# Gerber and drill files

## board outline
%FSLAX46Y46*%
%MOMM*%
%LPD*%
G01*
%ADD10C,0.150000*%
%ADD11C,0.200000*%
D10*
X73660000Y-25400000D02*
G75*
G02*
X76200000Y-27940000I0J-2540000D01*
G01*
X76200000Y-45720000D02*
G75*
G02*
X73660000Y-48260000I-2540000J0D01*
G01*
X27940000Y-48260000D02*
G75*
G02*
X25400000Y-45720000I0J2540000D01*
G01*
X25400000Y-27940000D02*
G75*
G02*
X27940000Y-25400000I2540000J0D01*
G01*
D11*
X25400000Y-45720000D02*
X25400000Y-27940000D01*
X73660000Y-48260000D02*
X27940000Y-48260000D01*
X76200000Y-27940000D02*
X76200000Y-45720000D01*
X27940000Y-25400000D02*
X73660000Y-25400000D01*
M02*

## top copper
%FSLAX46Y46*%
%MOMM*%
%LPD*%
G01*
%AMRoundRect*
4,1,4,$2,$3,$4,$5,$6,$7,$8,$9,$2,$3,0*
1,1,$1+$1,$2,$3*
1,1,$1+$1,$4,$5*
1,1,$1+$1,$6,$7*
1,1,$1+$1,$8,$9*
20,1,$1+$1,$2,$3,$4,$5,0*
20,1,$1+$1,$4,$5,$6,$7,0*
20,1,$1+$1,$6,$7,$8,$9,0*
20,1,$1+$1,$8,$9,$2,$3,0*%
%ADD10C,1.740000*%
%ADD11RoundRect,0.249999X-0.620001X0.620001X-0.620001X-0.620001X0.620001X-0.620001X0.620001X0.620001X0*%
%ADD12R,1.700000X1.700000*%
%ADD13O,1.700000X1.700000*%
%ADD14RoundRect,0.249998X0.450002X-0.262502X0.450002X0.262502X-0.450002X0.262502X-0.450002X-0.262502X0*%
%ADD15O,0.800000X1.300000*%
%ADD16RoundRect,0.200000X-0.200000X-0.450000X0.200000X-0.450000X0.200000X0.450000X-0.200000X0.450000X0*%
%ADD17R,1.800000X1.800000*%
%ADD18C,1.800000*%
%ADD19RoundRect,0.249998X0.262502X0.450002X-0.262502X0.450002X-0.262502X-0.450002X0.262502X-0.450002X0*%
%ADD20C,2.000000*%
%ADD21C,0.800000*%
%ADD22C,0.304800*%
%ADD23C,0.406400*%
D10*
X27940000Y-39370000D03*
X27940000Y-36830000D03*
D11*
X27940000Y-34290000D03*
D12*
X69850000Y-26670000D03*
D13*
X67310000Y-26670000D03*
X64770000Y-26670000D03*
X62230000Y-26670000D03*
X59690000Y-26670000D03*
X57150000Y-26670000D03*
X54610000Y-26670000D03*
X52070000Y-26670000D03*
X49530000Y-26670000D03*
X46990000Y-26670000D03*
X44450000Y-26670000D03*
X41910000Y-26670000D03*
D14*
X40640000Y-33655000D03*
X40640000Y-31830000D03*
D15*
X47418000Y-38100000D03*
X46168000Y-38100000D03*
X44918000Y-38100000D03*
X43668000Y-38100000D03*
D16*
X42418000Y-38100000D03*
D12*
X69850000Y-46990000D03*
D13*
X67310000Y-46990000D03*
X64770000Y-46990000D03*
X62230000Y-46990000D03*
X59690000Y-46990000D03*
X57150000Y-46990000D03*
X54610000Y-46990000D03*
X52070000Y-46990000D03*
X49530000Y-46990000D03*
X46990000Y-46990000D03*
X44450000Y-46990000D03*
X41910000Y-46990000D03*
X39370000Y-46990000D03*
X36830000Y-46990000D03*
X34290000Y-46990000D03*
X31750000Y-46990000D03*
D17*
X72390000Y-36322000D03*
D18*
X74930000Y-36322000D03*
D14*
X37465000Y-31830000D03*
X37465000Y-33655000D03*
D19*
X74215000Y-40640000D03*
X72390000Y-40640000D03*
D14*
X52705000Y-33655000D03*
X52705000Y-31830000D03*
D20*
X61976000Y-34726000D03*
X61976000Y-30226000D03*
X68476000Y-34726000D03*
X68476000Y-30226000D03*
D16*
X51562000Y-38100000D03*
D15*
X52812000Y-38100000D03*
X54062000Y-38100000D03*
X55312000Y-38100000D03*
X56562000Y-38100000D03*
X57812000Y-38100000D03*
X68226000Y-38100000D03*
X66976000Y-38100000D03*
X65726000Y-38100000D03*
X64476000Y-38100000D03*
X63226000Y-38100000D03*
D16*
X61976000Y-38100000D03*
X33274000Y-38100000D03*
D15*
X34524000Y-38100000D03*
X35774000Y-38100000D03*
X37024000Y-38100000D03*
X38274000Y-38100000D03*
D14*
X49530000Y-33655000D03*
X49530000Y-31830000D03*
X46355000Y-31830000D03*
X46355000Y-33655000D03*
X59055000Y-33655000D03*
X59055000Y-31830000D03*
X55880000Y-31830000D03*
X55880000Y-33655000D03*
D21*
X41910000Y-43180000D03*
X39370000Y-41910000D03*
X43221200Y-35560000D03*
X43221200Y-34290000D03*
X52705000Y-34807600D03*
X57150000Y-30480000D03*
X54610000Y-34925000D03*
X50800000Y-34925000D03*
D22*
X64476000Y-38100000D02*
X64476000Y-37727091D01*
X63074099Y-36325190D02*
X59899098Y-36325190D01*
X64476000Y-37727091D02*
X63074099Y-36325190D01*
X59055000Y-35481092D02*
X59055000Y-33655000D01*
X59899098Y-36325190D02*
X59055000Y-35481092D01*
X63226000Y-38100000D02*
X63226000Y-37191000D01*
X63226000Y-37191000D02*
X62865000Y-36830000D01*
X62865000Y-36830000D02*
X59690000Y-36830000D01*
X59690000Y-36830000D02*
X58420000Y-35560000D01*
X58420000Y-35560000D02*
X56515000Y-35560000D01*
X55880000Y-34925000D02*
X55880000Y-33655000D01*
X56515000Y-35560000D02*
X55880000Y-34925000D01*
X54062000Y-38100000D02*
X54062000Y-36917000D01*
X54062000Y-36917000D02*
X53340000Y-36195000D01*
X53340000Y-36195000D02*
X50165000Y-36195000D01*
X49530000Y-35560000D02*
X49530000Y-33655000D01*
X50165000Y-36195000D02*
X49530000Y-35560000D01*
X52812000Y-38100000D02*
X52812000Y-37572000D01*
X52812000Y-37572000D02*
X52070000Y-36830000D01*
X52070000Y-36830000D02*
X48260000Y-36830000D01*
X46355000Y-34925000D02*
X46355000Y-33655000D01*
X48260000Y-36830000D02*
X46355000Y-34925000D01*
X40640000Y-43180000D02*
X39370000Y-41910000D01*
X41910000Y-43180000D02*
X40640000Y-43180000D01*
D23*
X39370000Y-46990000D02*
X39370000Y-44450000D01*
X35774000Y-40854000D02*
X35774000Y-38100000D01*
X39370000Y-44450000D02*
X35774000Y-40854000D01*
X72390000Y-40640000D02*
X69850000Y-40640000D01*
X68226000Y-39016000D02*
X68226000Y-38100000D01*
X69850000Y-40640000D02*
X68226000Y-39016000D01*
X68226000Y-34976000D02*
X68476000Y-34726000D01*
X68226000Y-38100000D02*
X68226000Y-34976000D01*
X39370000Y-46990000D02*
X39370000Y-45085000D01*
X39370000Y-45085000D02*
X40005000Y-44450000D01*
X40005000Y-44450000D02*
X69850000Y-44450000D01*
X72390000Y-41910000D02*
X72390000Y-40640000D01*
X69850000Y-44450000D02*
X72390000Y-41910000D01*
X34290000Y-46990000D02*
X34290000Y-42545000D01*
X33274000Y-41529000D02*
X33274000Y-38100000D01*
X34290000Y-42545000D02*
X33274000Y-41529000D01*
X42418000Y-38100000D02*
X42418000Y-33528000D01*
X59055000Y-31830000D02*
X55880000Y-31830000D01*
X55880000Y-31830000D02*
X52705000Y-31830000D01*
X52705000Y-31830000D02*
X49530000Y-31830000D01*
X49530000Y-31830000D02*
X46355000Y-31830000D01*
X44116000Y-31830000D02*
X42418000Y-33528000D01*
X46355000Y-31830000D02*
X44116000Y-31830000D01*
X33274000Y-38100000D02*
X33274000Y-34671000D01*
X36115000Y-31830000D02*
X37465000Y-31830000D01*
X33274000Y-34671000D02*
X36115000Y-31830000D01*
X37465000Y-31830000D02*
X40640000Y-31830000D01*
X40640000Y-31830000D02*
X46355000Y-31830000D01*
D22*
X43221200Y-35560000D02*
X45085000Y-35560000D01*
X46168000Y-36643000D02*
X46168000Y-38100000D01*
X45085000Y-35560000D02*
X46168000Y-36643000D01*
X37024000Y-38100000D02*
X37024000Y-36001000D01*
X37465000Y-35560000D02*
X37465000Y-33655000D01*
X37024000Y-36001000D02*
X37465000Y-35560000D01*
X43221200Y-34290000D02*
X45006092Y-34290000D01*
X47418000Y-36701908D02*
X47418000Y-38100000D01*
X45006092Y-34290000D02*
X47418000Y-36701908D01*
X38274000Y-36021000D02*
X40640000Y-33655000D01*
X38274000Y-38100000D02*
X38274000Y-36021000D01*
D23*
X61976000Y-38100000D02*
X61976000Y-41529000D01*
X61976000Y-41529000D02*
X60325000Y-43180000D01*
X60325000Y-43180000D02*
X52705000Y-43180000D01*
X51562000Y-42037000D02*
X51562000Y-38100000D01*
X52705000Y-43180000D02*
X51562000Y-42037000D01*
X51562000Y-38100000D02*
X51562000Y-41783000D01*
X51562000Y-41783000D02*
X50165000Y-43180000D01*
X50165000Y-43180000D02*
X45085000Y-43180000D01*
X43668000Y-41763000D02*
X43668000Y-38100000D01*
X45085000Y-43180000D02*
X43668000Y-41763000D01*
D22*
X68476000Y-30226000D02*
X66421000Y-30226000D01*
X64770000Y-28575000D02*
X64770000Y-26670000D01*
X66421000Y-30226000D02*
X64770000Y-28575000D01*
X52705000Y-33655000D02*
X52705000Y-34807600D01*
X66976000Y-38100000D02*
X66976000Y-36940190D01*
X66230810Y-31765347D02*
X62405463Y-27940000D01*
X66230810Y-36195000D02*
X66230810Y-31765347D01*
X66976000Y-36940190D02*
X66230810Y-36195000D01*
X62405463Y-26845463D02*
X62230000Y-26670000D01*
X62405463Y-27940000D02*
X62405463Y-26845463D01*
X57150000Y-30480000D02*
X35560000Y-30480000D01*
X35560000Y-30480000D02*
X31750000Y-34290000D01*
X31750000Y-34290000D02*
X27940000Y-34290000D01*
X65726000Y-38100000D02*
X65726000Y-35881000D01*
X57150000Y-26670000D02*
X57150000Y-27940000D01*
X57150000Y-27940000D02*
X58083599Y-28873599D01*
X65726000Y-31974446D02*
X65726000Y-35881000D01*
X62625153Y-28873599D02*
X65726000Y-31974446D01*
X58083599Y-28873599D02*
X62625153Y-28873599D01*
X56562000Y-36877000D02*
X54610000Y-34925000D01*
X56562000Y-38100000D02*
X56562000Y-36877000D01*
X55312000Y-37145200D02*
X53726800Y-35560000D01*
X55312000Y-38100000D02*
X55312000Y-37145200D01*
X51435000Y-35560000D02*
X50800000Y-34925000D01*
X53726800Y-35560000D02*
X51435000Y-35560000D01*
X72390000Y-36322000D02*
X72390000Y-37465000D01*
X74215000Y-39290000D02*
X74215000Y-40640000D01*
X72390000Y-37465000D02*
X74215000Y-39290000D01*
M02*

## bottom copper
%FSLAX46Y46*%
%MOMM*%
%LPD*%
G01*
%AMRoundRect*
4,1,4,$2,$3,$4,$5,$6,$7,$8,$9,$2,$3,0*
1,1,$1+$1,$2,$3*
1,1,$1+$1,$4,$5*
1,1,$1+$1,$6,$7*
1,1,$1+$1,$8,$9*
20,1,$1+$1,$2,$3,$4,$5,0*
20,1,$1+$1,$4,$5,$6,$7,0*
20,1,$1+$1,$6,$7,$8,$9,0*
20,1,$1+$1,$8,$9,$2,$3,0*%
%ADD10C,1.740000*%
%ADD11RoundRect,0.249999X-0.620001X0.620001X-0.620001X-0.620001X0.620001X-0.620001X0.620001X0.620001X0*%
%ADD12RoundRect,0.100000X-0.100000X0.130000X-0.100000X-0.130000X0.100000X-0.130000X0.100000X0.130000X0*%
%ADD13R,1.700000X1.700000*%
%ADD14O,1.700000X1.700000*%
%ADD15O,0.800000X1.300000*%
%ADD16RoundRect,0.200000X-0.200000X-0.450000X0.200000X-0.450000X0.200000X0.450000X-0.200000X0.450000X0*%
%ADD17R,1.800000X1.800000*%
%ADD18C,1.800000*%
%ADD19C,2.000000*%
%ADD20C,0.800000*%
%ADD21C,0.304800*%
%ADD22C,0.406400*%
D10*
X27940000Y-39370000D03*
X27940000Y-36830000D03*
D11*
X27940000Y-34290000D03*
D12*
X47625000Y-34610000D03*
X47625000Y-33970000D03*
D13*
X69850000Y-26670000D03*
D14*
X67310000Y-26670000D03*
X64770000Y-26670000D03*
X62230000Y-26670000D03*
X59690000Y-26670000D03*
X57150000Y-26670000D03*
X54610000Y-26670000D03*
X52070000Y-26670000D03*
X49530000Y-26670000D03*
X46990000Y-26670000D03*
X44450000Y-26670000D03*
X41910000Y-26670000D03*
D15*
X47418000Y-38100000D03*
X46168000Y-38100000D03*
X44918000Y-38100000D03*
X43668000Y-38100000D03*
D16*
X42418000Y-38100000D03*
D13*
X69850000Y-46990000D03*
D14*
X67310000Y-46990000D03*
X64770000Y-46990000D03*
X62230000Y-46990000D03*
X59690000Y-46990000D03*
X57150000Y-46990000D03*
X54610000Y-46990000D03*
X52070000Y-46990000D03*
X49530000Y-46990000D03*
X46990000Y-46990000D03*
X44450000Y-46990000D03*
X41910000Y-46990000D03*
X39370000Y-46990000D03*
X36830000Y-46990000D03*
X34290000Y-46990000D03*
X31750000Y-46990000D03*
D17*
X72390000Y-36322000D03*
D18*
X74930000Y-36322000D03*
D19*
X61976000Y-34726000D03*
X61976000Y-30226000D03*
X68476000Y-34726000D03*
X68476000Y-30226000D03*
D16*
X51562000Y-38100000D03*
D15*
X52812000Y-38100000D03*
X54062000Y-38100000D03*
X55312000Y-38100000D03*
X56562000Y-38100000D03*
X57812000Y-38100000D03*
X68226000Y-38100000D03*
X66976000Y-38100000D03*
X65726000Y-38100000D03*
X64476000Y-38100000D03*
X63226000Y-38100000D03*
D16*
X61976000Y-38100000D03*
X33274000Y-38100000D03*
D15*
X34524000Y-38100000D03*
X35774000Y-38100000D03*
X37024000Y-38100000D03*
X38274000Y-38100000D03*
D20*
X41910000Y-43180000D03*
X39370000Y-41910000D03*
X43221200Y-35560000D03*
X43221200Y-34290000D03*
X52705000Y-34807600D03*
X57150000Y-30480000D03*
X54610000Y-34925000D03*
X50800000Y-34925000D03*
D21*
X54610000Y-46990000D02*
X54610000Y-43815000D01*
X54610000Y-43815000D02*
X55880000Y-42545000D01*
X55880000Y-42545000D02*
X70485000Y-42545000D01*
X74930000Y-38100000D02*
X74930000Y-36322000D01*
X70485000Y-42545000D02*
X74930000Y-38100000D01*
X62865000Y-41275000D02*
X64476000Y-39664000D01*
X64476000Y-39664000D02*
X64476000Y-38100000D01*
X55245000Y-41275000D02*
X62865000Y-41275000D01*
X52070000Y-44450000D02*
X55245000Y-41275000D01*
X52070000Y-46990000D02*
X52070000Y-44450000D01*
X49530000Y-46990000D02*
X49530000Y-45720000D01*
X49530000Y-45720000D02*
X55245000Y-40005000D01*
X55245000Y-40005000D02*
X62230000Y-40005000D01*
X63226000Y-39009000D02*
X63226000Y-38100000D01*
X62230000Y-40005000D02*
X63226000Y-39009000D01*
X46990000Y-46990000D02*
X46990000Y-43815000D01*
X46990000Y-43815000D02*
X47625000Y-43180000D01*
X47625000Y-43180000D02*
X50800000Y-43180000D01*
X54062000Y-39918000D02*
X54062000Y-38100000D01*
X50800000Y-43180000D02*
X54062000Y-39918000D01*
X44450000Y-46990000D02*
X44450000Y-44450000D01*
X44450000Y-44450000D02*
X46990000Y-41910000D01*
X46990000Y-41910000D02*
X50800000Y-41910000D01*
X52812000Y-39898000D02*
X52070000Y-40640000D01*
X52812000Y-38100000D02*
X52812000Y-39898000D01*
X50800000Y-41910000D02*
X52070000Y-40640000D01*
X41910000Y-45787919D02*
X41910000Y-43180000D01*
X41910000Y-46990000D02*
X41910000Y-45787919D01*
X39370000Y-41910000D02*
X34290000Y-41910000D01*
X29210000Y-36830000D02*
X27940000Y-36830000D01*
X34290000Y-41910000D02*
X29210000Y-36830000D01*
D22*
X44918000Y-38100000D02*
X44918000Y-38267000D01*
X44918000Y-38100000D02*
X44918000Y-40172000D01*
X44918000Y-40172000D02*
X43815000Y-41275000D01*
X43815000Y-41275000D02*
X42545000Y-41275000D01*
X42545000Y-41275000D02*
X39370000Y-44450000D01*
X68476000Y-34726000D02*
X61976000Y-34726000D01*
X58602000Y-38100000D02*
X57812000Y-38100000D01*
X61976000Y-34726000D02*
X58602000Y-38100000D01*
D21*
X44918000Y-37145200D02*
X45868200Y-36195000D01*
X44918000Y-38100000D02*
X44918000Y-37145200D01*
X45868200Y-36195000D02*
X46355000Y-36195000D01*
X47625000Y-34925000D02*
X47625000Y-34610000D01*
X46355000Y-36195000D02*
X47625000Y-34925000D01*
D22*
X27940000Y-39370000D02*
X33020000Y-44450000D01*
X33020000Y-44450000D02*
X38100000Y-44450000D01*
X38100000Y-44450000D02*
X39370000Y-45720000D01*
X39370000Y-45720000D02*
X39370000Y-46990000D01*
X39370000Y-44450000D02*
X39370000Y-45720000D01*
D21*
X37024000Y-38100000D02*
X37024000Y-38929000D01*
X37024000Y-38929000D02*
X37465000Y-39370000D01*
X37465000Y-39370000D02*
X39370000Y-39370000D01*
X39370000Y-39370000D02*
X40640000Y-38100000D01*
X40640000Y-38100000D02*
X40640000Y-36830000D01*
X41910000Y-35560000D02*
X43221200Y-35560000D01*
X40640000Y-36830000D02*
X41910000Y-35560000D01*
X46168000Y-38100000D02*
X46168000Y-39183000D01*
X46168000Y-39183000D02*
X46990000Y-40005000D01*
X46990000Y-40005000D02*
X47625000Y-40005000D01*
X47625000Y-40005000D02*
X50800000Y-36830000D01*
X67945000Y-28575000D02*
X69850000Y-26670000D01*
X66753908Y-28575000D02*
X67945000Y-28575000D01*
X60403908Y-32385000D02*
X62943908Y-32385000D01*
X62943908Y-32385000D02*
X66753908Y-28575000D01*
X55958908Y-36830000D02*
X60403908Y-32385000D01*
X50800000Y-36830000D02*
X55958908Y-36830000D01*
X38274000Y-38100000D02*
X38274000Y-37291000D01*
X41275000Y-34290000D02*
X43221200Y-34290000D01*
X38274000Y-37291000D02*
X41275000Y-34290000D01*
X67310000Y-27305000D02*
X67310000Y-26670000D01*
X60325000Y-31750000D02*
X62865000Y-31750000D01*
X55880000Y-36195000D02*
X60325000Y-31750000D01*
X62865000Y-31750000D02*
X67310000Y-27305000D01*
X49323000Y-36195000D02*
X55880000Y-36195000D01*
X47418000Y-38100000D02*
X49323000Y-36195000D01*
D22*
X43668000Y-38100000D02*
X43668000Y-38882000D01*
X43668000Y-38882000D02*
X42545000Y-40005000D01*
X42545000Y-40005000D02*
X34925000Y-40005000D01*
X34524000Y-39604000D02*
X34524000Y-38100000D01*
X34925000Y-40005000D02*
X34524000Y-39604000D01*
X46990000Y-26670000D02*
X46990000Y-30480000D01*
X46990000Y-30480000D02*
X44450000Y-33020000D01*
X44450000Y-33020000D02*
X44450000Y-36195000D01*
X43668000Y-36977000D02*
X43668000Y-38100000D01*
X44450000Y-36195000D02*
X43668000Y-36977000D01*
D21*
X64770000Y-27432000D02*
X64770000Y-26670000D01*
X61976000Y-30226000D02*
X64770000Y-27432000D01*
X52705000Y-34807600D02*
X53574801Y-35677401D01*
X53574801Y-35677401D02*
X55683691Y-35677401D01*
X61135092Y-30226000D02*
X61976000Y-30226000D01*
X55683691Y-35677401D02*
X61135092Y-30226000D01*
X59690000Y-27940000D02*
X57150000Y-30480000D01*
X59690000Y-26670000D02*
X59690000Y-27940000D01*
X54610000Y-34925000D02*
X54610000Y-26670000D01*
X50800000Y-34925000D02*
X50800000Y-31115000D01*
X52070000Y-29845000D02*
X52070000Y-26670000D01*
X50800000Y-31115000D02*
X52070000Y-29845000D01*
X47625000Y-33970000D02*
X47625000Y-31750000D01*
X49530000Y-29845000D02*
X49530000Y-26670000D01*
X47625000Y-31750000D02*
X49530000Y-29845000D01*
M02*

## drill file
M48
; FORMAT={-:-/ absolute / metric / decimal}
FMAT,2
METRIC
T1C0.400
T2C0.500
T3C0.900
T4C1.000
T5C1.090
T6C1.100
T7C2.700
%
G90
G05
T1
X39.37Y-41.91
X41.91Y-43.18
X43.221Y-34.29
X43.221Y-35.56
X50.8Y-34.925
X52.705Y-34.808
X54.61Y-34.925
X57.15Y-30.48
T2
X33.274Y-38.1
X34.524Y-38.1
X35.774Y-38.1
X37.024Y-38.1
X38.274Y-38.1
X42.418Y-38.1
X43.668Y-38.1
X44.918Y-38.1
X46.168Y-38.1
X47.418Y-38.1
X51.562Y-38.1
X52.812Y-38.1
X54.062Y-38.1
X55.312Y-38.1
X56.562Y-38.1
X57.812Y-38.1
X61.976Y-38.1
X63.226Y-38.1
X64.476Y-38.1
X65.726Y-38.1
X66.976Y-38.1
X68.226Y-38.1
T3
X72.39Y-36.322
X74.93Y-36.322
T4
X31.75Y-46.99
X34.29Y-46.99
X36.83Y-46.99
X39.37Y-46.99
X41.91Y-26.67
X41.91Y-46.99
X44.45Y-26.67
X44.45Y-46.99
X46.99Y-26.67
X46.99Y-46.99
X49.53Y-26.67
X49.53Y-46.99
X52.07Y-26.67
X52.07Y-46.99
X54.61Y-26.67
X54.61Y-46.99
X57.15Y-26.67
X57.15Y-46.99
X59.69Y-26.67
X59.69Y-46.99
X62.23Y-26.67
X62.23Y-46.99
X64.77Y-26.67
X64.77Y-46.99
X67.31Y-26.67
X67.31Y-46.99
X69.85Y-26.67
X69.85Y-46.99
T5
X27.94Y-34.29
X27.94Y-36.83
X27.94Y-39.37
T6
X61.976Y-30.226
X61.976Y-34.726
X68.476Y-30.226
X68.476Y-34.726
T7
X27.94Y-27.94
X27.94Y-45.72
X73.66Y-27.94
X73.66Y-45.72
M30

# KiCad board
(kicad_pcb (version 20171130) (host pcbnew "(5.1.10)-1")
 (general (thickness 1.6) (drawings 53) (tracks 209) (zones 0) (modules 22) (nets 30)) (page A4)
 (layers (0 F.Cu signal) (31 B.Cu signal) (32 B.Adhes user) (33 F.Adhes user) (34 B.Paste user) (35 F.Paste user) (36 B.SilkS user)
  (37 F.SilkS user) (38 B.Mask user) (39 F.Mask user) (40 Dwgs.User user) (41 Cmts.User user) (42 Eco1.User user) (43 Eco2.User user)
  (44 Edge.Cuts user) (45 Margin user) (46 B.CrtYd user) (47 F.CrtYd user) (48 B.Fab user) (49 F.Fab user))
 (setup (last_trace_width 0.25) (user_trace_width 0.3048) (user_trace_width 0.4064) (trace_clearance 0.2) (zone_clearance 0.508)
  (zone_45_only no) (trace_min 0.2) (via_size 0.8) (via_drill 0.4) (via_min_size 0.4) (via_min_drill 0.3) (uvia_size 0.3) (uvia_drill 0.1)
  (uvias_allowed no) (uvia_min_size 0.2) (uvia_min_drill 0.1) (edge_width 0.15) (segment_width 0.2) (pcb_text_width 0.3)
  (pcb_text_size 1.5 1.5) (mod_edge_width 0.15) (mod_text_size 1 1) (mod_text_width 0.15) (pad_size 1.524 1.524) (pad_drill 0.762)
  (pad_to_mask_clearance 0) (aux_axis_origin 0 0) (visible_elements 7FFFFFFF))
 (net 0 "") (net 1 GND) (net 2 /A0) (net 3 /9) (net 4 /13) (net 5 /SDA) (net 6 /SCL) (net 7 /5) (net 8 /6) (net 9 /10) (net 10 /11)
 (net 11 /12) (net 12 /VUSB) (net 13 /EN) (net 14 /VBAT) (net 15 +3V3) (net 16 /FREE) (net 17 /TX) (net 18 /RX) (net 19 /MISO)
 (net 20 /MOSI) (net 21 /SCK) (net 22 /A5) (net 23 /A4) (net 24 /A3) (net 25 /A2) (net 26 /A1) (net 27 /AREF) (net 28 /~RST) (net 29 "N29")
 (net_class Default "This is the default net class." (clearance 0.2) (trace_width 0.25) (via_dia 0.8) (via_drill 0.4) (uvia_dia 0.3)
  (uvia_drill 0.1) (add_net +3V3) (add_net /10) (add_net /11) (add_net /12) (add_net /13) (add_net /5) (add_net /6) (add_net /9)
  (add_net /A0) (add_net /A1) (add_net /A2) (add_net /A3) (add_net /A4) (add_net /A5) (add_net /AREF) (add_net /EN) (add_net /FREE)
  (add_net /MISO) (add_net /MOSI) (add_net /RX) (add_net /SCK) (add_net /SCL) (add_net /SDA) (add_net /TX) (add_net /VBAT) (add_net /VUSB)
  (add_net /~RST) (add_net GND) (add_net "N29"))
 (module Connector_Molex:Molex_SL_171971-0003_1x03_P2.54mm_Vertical (layer F.Cu) (at 27.94 34.29 270)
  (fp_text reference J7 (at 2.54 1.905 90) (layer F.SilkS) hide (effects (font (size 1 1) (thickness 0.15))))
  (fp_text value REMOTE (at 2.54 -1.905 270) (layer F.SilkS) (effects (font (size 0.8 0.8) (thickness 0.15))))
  (pad 3 thru_hole circle (at 5.08 0 270) (size 1.74 1.74) (drill 1.09) (layers *.Cu *.Mask) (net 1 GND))
  (pad 2 thru_hole circle (at 2.54 0 270) (size 1.74 1.74) (drill 1.09) (layers *.Cu *.Mask) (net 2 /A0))
  (pad 1 thru_hole roundrect (at 0 0 270) (size 1.74 1.74) (drill 1.09) (layers *.Cu *.Mask) (roundrect_rratio 0.1436775862068966)
   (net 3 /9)))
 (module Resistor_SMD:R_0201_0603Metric (layer B.Cu) (at 47.625 34.29 270)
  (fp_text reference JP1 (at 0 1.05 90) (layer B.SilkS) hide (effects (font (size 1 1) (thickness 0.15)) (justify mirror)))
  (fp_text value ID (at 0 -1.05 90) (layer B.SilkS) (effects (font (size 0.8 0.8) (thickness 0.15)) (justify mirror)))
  (pad 2 smd roundrect (at 0.32 0 270) (size 0.46 0.4) (layers B.Cu B.Mask) (roundrect_rratio 0.25) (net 1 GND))
  (pad 1 smd roundrect (at -0.32 0 270) (size 0.46 0.4) (layers B.Cu B.Mask) (roundrect_rratio 0.25) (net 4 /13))
  (pad "" smd roundrect (at 0.345 0 270) (size 0.318 0.36) (layers B.Paste) (roundrect_rratio 0.25))
  (pad "" smd roundrect (at -0.345 0 270) (size 0.318 0.36) (layers B.Paste) (roundrect_rratio 0.25)))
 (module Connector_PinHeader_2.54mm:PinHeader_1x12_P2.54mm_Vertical (layer B.Cu) (at 69.85 26.67 90)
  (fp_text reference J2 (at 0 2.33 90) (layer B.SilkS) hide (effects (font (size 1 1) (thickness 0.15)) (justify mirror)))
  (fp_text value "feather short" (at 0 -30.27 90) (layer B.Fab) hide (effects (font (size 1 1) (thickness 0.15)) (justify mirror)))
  (pad 1 thru_hole rect (at 0 0 90) (size 1.7 1.7) (drill 1) (layers *.Cu *.Mask) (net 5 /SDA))
  (pad 2 thru_hole oval (at 0 -2.54 90) (size 1.7 1.7) (drill 1) (layers *.Cu *.Mask) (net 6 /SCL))
  (pad 3 thru_hole oval (at 0 -5.08 90) (size 1.7 1.7) (drill 1) (layers *.Cu *.Mask) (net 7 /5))
  (pad 4 thru_hole oval (at 0 -7.62 90) (size 1.7 1.7) (drill 1) (layers *.Cu *.Mask) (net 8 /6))
  (pad 5 thru_hole oval (at 0 -10.16 90) (size 1.7 1.7) (drill 1) (layers *.Cu *.Mask) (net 3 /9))
  (pad 6 thru_hole oval (at 0 -12.7 90) (size 1.7 1.7) (drill 1) (layers *.Cu *.Mask) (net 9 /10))
  (pad 7 thru_hole oval (at 0 -15.24 90) (size 1.7 1.7) (drill 1) (layers *.Cu *.Mask) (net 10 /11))
  (pad 8 thru_hole oval (at 0 -17.78 90) (size 1.7 1.7) (drill 1) (layers *.Cu *.Mask) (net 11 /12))
  (pad 9 thru_hole oval (at 0 -20.32 90) (size 1.7 1.7) (drill 1) (layers *.Cu *.Mask) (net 4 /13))
  (pad 10 thru_hole oval (at 0 -22.86 90) (size 1.7 1.7) (drill 1) (layers *.Cu *.Mask) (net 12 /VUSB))
  (pad 11 thru_hole oval (at 0 -25.4 90) (size 1.7 1.7) (drill 1) (layers *.Cu *.Mask) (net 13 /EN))
  (pad 12 thru_hole oval (at 0 -27.94 90) (size 1.7 1.7) (drill 1) (layers *.Cu *.Mask) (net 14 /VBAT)))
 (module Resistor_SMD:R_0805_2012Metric (layer F.Cu) (at 40.64 32.7425 90)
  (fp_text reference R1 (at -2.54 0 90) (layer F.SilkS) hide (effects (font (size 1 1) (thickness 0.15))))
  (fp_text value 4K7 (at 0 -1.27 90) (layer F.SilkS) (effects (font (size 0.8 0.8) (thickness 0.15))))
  (pad 1 smd roundrect (at -0.9125 0 90) (size 1.025 1.4) (layers F.Cu F.Paste F.Mask) (roundrect_rratio 0.2439004878048781) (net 6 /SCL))
  (pad 2 smd roundrect (at 0.9125 0 90) (size 1.025 1.4) (layers F.Cu F.Paste F.Mask) (roundrect_rratio 0.2439004878048781) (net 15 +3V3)))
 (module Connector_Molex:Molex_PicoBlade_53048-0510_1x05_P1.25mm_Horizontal (layer F.Cu) (at 42.418 38.1)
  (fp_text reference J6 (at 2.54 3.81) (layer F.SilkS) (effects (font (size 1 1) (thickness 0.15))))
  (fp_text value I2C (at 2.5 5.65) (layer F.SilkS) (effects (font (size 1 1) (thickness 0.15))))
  (pad 5 thru_hole oval (at 5 0) (size 0.8 1.3) (drill 0.5) (layers *.Cu *.Mask) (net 6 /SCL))
  (pad 4 thru_hole oval (at 3.75 0) (size 0.8 1.3) (drill 0.5) (layers *.Cu *.Mask) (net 5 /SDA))
  (pad 3 thru_hole oval (at 2.5 0) (size 0.8 1.3) (drill 0.5) (layers *.Cu *.Mask) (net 1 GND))
  (pad 2 thru_hole oval (at 1.25 0) (size 0.8 1.3) (drill 0.5) (layers *.Cu *.Mask) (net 12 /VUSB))
  (pad 1 thru_hole roundrect (at 0 0) (size 0.8 1.3) (drill 0.5) (layers *.Cu *.Mask) (roundrect_rratio 0.25) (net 15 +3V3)))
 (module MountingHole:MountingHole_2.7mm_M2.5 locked (layer F.Cu) (at 73.66 27.94)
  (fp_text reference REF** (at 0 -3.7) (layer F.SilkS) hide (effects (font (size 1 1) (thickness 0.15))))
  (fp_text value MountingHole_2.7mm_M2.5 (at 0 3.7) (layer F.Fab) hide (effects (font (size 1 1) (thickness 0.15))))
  (pad 1 np_thru_hole circle (at 0 0) (size 2.7 2.7) (drill 2.7) (layers *.Cu *.Mask)))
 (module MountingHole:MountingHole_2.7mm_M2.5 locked (layer F.Cu) (at 73.66 45.72)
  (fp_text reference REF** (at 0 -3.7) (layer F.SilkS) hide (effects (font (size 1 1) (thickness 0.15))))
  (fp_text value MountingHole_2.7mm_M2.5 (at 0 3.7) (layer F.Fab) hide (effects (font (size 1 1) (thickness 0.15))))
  (pad 1 np_thru_hole circle (at 0 0) (size 2.7 2.7) (drill 2.7) (layers *.Cu *.Mask)))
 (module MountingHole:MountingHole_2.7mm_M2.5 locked (layer F.Cu) (at 27.94 45.72)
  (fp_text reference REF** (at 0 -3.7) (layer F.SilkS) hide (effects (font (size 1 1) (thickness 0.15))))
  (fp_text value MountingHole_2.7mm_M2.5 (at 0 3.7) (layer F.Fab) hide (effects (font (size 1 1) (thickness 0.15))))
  (pad 1 np_thru_hole circle (at 0 0) (size 2.7 2.7) (drill 2.7) (layers *.Cu *.Mask)))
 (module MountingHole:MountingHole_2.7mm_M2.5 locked (layer F.Cu) (at 27.94 27.94)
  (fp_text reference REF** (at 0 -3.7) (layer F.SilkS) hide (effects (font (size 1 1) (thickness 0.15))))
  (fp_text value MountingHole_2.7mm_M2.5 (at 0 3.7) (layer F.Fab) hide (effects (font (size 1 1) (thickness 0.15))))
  (pad 1 np_thru_hole circle (at 0 0) (size 2.7 2.7) (drill 2.7) (layers *.Cu *.Mask)))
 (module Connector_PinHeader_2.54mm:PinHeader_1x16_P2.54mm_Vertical (layer B.Cu) (at 69.85 46.99 90)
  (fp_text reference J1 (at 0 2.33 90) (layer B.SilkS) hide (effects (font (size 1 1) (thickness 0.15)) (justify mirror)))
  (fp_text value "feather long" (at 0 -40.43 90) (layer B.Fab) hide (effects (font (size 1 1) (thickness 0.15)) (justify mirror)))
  (pad 1 thru_hole rect (at 0 0 90) (size 1.7 1.7) (drill 1) (layers *.Cu *.Mask) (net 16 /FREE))
  (pad 2 thru_hole oval (at 0 -2.54 90) (size 1.7 1.7) (drill 1) (layers *.Cu *.Mask) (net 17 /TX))
  (pad 3 thru_hole oval (at 0 -5.08 90) (size 1.7 1.7) (drill 1) (layers *.Cu *.Mask) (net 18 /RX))
  (pad 4 thru_hole oval (at 0 -7.62 90) (size 1.7 1.7) (drill 1) (layers *.Cu *.Mask) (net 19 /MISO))
  (pad 5 thru_hole oval (at 0 -10.16 90) (size 1.7 1.7) (drill 1) (layers *.Cu *.Mask) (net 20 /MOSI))
  (pad 6 thru_hole oval (at 0 -12.7 90) (size 1.7 1.7) (drill 1) (layers *.Cu *.Mask) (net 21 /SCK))
  (pad 7 thru_hole oval (at 0 -15.24 90) (size 1.7 1.7) (drill 1) (layers *.Cu *.Mask) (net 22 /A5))
  (pad 8 thru_hole oval (at 0 -17.78 90) (size 1.7 1.7) (drill 1) (layers *.Cu *.Mask) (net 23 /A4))
  (pad 9 thru_hole oval (at 0 -20.32 90) (size 1.7 1.7) (drill 1) (layers *.Cu *.Mask) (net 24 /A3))
  (pad 10 thru_hole oval (at 0 -22.86 90) (size 1.7 1.7) (drill 1) (layers *.Cu *.Mask) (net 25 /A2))
  (pad 11 thru_hole oval (at 0 -25.4 90) (size 1.7 1.7) (drill 1) (layers *.Cu *.Mask) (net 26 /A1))
  (pad 12 thru_hole oval (at 0 -27.94 90) (size 1.7 1.7) (drill 1) (layers *.Cu *.Mask) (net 2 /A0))
  (pad 13 thru_hole oval (at 0 -30.48 90) (size 1.7 1.7) (drill 1) (layers *.Cu *.Mask) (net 1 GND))
  (pad 14 thru_hole oval (at 0 -33.02 90) (size 1.7 1.7) (drill 1) (layers *.Cu *.Mask) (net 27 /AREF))
  (pad 15 thru_hole oval (at 0 -35.56 90) (size 1.7 1.7) (drill 1) (layers *.Cu *.Mask) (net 15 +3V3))
  (pad 16 thru_hole oval (at 0 -38.1 90) (size 1.7 1.7) (drill 1) (layers *.Cu *.Mask) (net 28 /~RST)))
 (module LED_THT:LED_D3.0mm (layer F.Cu) (at 72.39 36.322)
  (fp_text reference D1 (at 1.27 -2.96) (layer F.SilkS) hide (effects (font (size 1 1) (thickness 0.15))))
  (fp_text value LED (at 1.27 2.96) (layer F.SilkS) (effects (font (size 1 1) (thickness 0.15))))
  (pad 1 thru_hole rect (at 0 0) (size 1.8 1.8) (drill 0.9) (layers *.Cu *.Mask) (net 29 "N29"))
  (pad 2 thru_hole circle (at 2.54 0) (size 1.8 1.8) (drill 0.9) (layers *.Cu *.Mask) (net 22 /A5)))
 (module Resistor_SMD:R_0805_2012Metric (layer F.Cu) (at 37.465 32.7425 90)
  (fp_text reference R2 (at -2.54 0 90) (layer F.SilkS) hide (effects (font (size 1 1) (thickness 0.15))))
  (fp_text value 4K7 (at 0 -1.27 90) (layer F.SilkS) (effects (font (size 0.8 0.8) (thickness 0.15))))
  (pad 2 smd roundrect (at 0.9125 0 90) (size 1.025 1.4) (layers F.Cu F.Paste F.Mask) (roundrect_rratio 0.2439004878048781) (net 15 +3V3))
  (pad 1 smd roundrect (at -0.9125 0 90) (size 1.025 1.4) (layers F.Cu F.Paste F.Mask) (roundrect_rratio 0.2439004878048781) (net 5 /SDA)))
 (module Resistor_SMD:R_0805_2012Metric (layer F.Cu) (at 73.3025 40.64 180)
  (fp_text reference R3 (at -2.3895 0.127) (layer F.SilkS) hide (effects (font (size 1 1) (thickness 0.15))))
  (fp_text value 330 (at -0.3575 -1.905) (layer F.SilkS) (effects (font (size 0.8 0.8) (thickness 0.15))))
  (pad 1 smd roundrect (at -0.9125 0 180) (size 1.025 1.4) (layers F.Cu F.Paste F.Mask) (roundrect_rratio 0.2439004878048781) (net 29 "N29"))
  (pad 2 smd roundrect (at 0.9125 0 180) (size 1.025 1.4) (layers F.Cu F.Paste F.Mask) (roundrect_rratio 0.2439004878048781) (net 1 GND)))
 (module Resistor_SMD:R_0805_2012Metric (layer F.Cu) (at 52.705 32.7425 90)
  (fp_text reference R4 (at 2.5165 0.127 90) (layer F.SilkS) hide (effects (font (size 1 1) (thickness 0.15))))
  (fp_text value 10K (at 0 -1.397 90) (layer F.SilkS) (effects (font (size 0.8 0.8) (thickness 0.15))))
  (pad 1 smd roundrect (at -0.9125 0 90) (size 1.025 1.4) (layers F.Cu F.Paste F.Mask) (roundrect_rratio 0.2439004878048781) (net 7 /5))
  (pad 2 smd roundrect (at 0.9125 0 90) (size 1.025 1.4) (layers F.Cu F.Paste F.Mask) (roundrect_rratio 0.2439004878048781) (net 15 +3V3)))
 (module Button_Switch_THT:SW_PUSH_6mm (layer F.Cu) (at 61.976 30.226)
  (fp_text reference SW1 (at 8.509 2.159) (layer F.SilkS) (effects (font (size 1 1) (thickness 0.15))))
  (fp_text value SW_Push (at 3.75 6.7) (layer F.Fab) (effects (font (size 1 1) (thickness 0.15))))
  (pad 2 thru_hole circle (at 0 4.5 90) (size 2 2) (drill 1.1) (layers *.Cu *.Mask) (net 1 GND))
  (pad 1 thru_hole circle (at 0 0 90) (size 2 2) (drill 1.1) (layers *.Cu *.Mask) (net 7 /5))
  (pad 2 thru_hole circle (at 6.5 4.5 90) (size 2 2) (drill 1.1) (layers *.Cu *.Mask) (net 1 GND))
  (pad 1 thru_hole circle (at 6.5 0 90) (size 2 2) (drill 1.1) (layers *.Cu *.Mask) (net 7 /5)))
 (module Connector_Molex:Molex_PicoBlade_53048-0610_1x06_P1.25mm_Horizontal (layer F.Cu) (at 51.562 38.1)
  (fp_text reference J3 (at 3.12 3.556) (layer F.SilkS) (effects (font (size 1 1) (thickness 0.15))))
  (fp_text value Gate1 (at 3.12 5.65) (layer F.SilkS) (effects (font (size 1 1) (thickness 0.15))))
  (pad 1 thru_hole roundrect (at 0 0) (size 0.8 1.3) (drill 0.5) (layers *.Cu *.Mask) (roundrect_rratio 0.25) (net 12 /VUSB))
  (pad 2 thru_hole oval (at 1.25 0) (size 0.8 1.3) (drill 0.5) (layers *.Cu *.Mask) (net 26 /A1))
  (pad 3 thru_hole oval (at 2.5 0) (size 0.8 1.3) (drill 0.5) (layers *.Cu *.Mask) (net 25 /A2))
  (pad 4 thru_hole oval (at 3.75 0) (size 0.8 1.3) (drill 0.5) (layers *.Cu *.Mask) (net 11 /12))
  (pad 5 thru_hole oval (at 5 0) (size 0.8 1.3) (drill 0.5) (layers *.Cu *.Mask) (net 10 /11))
  (pad 6 thru_hole oval (at 6.25 0) (size 0.8 1.3) (drill 0.5) (layers *.Cu *.Mask) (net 1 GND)))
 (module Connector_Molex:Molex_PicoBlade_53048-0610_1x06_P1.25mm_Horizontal (layer F.Cu) (at 61.976 38.1)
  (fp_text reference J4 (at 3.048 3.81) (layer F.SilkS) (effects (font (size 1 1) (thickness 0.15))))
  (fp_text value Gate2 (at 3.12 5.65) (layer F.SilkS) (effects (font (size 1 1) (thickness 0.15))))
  (pad 6 thru_hole oval (at 6.25 0) (size 0.8 1.3) (drill 0.5) (layers *.Cu *.Mask) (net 1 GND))
  (pad 5 thru_hole oval (at 5 0) (size 0.8 1.3) (drill 0.5) (layers *.Cu *.Mask) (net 8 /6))
  (pad 4 thru_hole oval (at 3.75 0) (size 0.8 1.3) (drill 0.5) (layers *.Cu *.Mask) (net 9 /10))
  (pad 3 thru_hole oval (at 2.5 0) (size 0.8 1.3) (drill 0.5) (layers *.Cu *.Mask) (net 23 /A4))
  (pad 2 thru_hole oval (at 1.25 0) (size 0.8 1.3) (drill 0.5) (layers *.Cu *.Mask) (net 24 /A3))
  (pad 1 thru_hole roundrect (at 0 0) (size 0.8 1.3) (drill 0.5) (layers *.Cu *.Mask) (roundrect_rratio 0.25) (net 12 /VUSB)))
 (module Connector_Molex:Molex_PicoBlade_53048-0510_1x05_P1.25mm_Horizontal (layer F.Cu) (at 33.274 38.1)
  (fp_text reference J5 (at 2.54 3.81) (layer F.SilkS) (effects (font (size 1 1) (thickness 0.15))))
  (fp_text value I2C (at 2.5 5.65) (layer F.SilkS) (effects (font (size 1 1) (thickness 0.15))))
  (pad 1 thru_hole roundrect (at 0 0) (size 0.8 1.3) (drill 0.5) (layers *.Cu *.Mask) (roundrect_rratio 0.25) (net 15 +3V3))
  (pad 2 thru_hole oval (at 1.25 0) (size 0.8 1.3) (drill 0.5) (layers *.Cu *.Mask) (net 12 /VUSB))
  (pad 3 thru_hole oval (at 2.5 0) (size 0.8 1.3) (drill 0.5) (layers *.Cu *.Mask) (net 1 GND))
  (pad 4 thru_hole oval (at 3.75 0) (size 0.8 1.3) (drill 0.5) (layers *.Cu *.Mask) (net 5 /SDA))
  (pad 5 thru_hole oval (at 5 0) (size 0.8 1.3) (drill 0.5) (layers *.Cu *.Mask) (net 6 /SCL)))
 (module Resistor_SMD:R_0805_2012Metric (layer F.Cu) (at 49.53 32.7425 90)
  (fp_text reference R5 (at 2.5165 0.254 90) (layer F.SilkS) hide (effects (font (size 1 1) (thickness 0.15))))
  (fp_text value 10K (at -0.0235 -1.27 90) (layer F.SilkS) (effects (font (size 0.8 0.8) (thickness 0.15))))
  (pad 1 smd roundrect (at -0.9125 0 90) (size 1.025 1.4) (layers F.Cu F.Paste F.Mask) (roundrect_rratio 0.2439004878048781) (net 25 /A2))
  (pad 2 smd roundrect (at 0.9125 0 90) (size 1.025 1.4) (layers F.Cu F.Paste F.Mask) (roundrect_rratio 0.2439004878048781) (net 15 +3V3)))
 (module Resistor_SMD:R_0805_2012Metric (layer F.Cu) (at 46.355 32.7425 90)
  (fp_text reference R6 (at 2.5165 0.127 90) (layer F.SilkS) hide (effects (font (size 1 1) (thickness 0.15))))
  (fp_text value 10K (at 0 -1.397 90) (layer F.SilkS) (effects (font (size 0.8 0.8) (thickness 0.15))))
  (pad 2 smd roundrect (at 0.9125 0 90) (size 1.025 1.4) (layers F.Cu F.Paste F.Mask) (roundrect_rratio 0.2439004878048781) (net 15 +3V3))
  (pad 1 smd roundrect (at -0.9125 0 90) (size 1.025 1.4) (layers F.Cu F.Paste F.Mask) (roundrect_rratio 0.2439004878048781) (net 26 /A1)))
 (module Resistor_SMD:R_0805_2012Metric (layer F.Cu) (at 59.055 32.7425 90)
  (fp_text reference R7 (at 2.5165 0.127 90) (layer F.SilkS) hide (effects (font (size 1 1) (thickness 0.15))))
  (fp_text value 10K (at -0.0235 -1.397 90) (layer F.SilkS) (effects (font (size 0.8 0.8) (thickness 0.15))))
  (pad 1 smd roundrect (at -0.9125 0 90) (size 1.025 1.4) (layers F.Cu F.Paste F.Mask) (roundrect_rratio 0.2439004878048781) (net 23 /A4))
  (pad 2 smd roundrect (at 0.9125 0 90) (size 1.025 1.4) (layers F.Cu F.Paste F.Mask) (roundrect_rratio 0.2439004878048781) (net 15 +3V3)))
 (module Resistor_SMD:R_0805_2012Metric (layer F.Cu) (at 55.88 32.7425 90)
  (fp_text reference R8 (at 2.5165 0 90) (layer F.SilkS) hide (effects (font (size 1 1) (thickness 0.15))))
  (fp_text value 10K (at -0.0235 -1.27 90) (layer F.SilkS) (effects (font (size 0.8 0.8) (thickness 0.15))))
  (pad 2 smd roundrect (at 0.9125 0 90) (size 1.025 1.4) (layers F.Cu F.Paste F.Mask) (roundrect_rratio 0.2439004878048781) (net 15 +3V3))
  (pad 1 smd roundrect (at -0.9125 0 90) (size 1.025 1.4) (layers F.Cu F.Paste F.Mask) (roundrect_rratio 0.2439004878048781) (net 24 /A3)))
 (gr_arc (start 73.66 27.94) (end 76.2 27.94) (angle -90) (layer Edge.Cuts) (width 0.15))
 (gr_arc (start 73.66 45.72) (end 73.66 48.26) (angle -90) (layer Edge.Cuts) (width 0.15))
 (gr_arc (start 27.94 45.72) (end 25.4 45.72) (angle -90) (layer Edge.Cuts) (width 0.15))
 (gr_arc (start 27.94 27.94) (end 27.94 25.4) (angle -90) (layer Edge.Cuts) (width 0.15))
 (gr_line (start 25.4 45.72) (end 25.4 27.94) (layer Edge.Cuts) (width 0.2))
 (gr_line (start 73.66 48.26) (end 27.94 48.26) (layer Edge.Cuts) (width 0.2))
 (gr_line (start 76.2 27.94) (end 76.2 45.72) (layer Edge.Cuts) (width 0.2))
 (gr_line (start 27.94 25.4) (end 73.66 25.4) (layer Edge.Cuts) (width 0.2))
 (segment (start 54.61 46.99) (end 54.61 43.815) (width 0.3048) (layer B.Cu) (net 22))
 (segment (start 54.61 43.815) (end 55.88 42.545) (width 0.3048) (layer B.Cu) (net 22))
 (segment (start 55.88 42.545) (end 70.485 42.545) (width 0.3048) (layer B.Cu) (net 22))
 (segment (start 74.93 38.1) (end 74.93 36.322) (width 0.3048) (layer B.Cu) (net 22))
 (segment (start 70.485 42.545) (end 74.93 38.1) (width 0.3048) (layer B.Cu) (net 22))
 (segment (start 62.865 41.275) (end 64.476 39.664) (width 0.3048) (layer B.Cu) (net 23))
 (segment (start 64.476 39.664) (end 64.476 38.1) (width 0.3048) (layer B.Cu) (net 23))
 (segment (start 55.245 41.275) (end 62.865 41.275) (width 0.3048) (layer B.Cu) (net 23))
 (segment (start 52.07 44.45) (end 55.245 41.275) (width 0.3048) (layer B.Cu) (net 23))
 (segment (start 52.07 46.99) (end 52.07 44.45) (width 0.3048) (layer B.Cu) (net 23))
 (segment (start 64.476 38.1) (end 64.476 37.727091) (width 0.3048) (layer F.Cu) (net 23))
 (segment (start 63.074099 36.32519) (end 59.899098 36.32519) (width 0.3048) (layer F.Cu) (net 23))
 (segment (start 64.476 37.727091) (end 63.074099 36.32519) (width 0.3048) (layer F.Cu) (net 23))
 (segment (start 59.055 35.481092) (end 59.055 33.655) (width 0.3048) (layer F.Cu) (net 23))
 (segment (start 59.899098 36.32519) (end 59.055 35.481092) (width 0.3048) (layer F.Cu) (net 23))
 (segment (start 49.53 46.99) (end 49.53 45.72) (width 0.3048) (layer B.Cu) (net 24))
 (segment (start 49.53 45.72) (end 55.245 40.005) (width 0.3048) (layer B.Cu) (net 24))
 (segment (start 55.245 40.005) (end 62.23 40.005) (width 0.3048) (layer B.Cu) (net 24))
 (segment (start 63.226 39.009) (end 63.226 38.1) (width 0.3048) (layer B.Cu) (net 24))
 (segment (start 62.23 40.005) (end 63.226 39.009) (width 0.3048) (layer B.Cu) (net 24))
 (segment (start 63.226 38.1) (end 63.226 37.191) (width 0.3048) (layer F.Cu) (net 24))
 (segment (start 63.226 37.191) (end 62.865 36.83) (width 0.3048) (layer F.Cu) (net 24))
 (segment (start 62.865 36.83) (end 59.69 36.83) (width 0.3048) (layer F.Cu) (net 24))
 (segment (start 59.69 36.83) (end 58.42 35.56) (width 0.3048) (layer F.Cu) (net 24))
 (segment (start 58.42 35.56) (end 56.515 35.56) (width 0.3048) (layer F.Cu) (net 24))
 (segment (start 55.88 34.925) (end 55.88 33.655) (width 0.3048) (layer F.Cu) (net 24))
 (segment (start 56.515 35.56) (end 55.88 34.925) (width 0.3048) (layer F.Cu) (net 24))
 (segment (start 46.99 46.99) (end 46.99 43.815) (width 0.3048) (layer B.Cu) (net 25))
 (segment (start 46.99 43.815) (end 47.625 43.18) (width 0.3048) (layer B.Cu) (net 25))
 (segment (start 47.625 43.18) (end 50.8 43.18) (width 0.3048) (layer B.Cu) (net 25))
 (segment (start 54.062 39.918) (end 54.062 38.1) (width 0.3048) (layer B.Cu) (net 25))
 (segment (start 50.8 43.18) (end 54.062 39.918) (width 0.3048) (layer B.Cu) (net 25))
 (segment (start 54.062 38.1) (end 54.062 36.917) (width 0.3048) (layer F.Cu) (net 25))
 (segment (start 54.062 36.917) (end 53.34 36.195) (width 0.3048) (layer F.Cu) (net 25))
 (segment (start 53.34 36.195) (end 50.165 36.195) (width 0.3048) (layer F.Cu) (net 25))
 (segment (start 49.53 35.56) (end 49.53 33.655) (width 0.3048) (layer F.Cu) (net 25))
 (segment (start 50.165 36.195) (end 49.53 35.56) (width 0.3048) (layer F.Cu) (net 25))
 (segment (start 44.45 46.99) (end 44.45 44.45) (width 0.3048) (layer B.Cu) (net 26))
 (segment (start 44.45 44.45) (end 46.99 41.91) (width 0.3048) (layer B.Cu) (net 26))
 (segment (start 46.99 41.91) (end 50.8 41.91) (width 0.3048) (layer B.Cu) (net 26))
 (segment (start 52.812 38.1) (end 52.812 37.572) (width 0.3048) (layer F.Cu) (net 26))
 (segment (start 52.812 37.572) (end 52.07 36.83) (width 0.3048) (layer F.Cu) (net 26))
 (segment (start 52.07 36.83) (end 48.26 36.83) (width 0.3048) (layer F.Cu) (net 26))
 (segment (start 46.355 34.925) (end 46.355 33.655) (width 0.3048) (layer F.Cu) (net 26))
 (segment (start 48.26 36.83) (end 46.355 34.925) (width 0.3048) (layer F.Cu) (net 26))
 (segment (start 52.812 39.898) (end 52.07 40.64) (width 0.3048) (layer B.Cu) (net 26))
 (segment (start 52.812 38.1) (end 52.812 39.898) (width 0.3048) (layer B.Cu) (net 26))
 (segment (start 50.8 41.91) (end 52.07 40.64) (width 0.3048) (layer B.Cu) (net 26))
 (via (at 41.91 43.18) (size 0.8) (drill 0.4) (layers F.Cu B.Cu) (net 2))
 (segment (start 41.91 45.787919) (end 41.91 43.18) (width 0.3048) (layer B.Cu) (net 2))
 (segment (start 41.91 46.99) (end 41.91 45.787919) (width 0.3048) (layer B.Cu) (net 2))
 (via (at 39.37 41.91) (size 0.8) (drill 0.4) (layers F.Cu B.Cu) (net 2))
 (segment (start 40.64 43.18) (end 39.37 41.91) (width 0.3048) (layer F.Cu) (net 2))
 (segment (start 41.91 43.18) (end 40.64 43.18) (width 0.3048) (layer F.Cu) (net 2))
 (segment (start 39.37 41.91) (end 34.29 41.91) (width 0.3048) (layer B.Cu) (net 2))
 (segment (start 29.21 36.83) (end 27.94 36.83) (width 0.3048) (layer B.Cu) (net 2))
 (segment (start 34.29 41.91) (end 29.21 36.83) (width 0.3048) (layer B.Cu) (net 2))
 (segment (start 39.37 46.99) (end 39.37 44.45) (width 0.4064) (layer F.Cu) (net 1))
 (segment (start 35.774 40.854) (end 35.774 38.1) (width 0.4064) (layer F.Cu) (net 1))
 (segment (start 39.37 44.45) (end 35.774 40.854) (width 0.4064) (layer F.Cu) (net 1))
 (segment (start 72.39 40.64) (end 69.85 40.64) (width 0.4064) (layer F.Cu) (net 1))
 (segment (start 68.226 39.016) (end 68.226 38.1) (width 0.4064) (layer F.Cu) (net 1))
 (segment (start 69.85 40.64) (end 68.226 39.016) (width 0.4064) (layer F.Cu) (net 1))
 (segment (start 68.226 34.976) (end 68.476 34.726) (width 0.4064) (layer F.Cu) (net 1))
 (segment (start 68.226 38.1) (end 68.226 34.976) (width 0.4064) (layer F.Cu) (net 1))
 (segment (start 44.918 38.1) (end 44.918 38.267) (width 0.4064) (layer B.Cu) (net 1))
 (segment (start 44.918 38.1) (end 44.918 40.172) (width 0.4064) (layer B.Cu) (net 1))
 (segment (start 44.918 40.172) (end 43.815 41.275) (width 0.4064) (layer B.Cu) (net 1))
 (segment (start 43.815 41.275) (end 42.545 41.275) (width 0.4064) (layer B.Cu) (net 1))
 (segment (start 42.545 41.275) (end 39.37 44.45) (width 0.4064) (layer B.Cu) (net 1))
 (segment (start 39.37 46.99) (end 39.37 45.085) (width 0.4064) (layer F.Cu) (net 1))
 (segment (start 39.37 45.085) (end 40.005 44.45) (width 0.4064) (layer F.Cu) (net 1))
 (segment (start 40.005 44.45) (end 69.85 44.45) (width 0.4064) (layer F.Cu) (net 1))
 (segment (start 72.39 41.91) (end 72.39 40.64) (width 0.4064) (layer F.Cu) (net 1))
 (segment (start 69.85 44.45) (end 72.39 41.91) (width 0.4064) (layer F.Cu) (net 1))
 (segment (start 68.476 34.726) (end 61.976 34.726) (width 0.4064) (layer B.Cu) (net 1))
 (segment (start 58.602 38.1) (end 57.812 38.1) (width 0.4064) (layer B.Cu) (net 1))
 (segment (start 61.976 34.726) (end 58.602 38.1) (width 0.4064) (layer B.Cu) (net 1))
 (segment (start 44.918 37.1452) (end 45.8682 36.195) (width 0.3048) (layer B.Cu) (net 1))
 (segment (start 44.918 38.1) (end 44.918 37.1452) (width 0.3048) (layer B.Cu) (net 1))
 (segment (start 45.8682 36.195) (end 46.355 36.195) (width 0.3048) (layer B.Cu) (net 1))
 (segment (start 47.625 34.925) (end 47.625 34.61) (width 0.3048) (layer B.Cu) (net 1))
 (segment (start 46.355 36.195) (end 47.625 34.925) (width 0.3048) (layer B.Cu) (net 1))
 (segment (start 27.94 39.37) (end 33.02 44.45) (width 0.4064) (layer B.Cu) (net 1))
 (segment (start 33.02 44.45) (end 38.1 44.45) (width 0.4064) (layer B.Cu) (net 1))
 (segment (start 38.1 44.45) (end 39.37 45.72) (width 0.4064) (layer B.Cu) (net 1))
 (segment (start 39.37 45.72) (end 39.37 46.99) (width 0.4064) (layer B.Cu) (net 1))
 (segment (start 39.37 44.45) (end 39.37 45.72) (width 0.4064) (layer B.Cu) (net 1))
 (segment (start 34.29 46.99) (end 34.29 42.545) (width 0.4064) (layer F.Cu) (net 15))
 (segment (start 33.274 41.529) (end 33.274 38.1) (width 0.4064) (layer F.Cu) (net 15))
 (segment (start 34.29 42.545) (end 33.274 41.529) (width 0.4064) (layer F.Cu) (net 15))
 (segment (start 42.418 38.1) (end 42.418 33.528) (width 0.4064) (layer F.Cu) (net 15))
 (segment (start 59.055 31.83) (end 55.88 31.83) (width 0.4064) (layer F.Cu) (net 15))
 (segment (start 55.88 31.83) (end 52.705 31.83) (width 0.4064) (layer F.Cu) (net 15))
 (segment (start 52.705 31.83) (end 49.53 31.83) (width 0.4064) (layer F.Cu) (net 15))
 (segment (start 49.53 31.83) (end 46.355 31.83) (width 0.4064) (layer F.Cu) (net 15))
 (segment (start 44.116 31.83) (end 42.418 33.528) (width 0.4064) (layer F.Cu) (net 15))
 (segment (start 46.355 31.83) (end 44.116 31.83) (width 0.4064) (layer F.Cu) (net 15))
 (segment (start 33.274 38.1) (end 33.274 34.671) (width 0.4064) (layer F.Cu) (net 15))
 (segment (start 36.115 31.83) (end 37.465 31.83) (width 0.4064) (layer F.Cu) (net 15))
 (segment (start 33.274 34.671) (end 36.115 31.83) (width 0.4064) (layer F.Cu) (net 15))
 (segment (start 37.465 31.83) (end 40.64 31.83) (width 0.4064) (layer F.Cu) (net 15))
 (segment (start 40.64 31.83) (end 46.355 31.83) (width 0.4064) (layer F.Cu) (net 15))
 (via (at 43.2212 35.56) (size 0.8) (drill 0.4) (layers F.Cu B.Cu) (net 5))
 (segment (start 43.2212 35.56) (end 45.085 35.56) (width 0.3048) (layer F.Cu) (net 5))
 (segment (start 46.168 36.643) (end 46.168 38.1) (width 0.3048) (layer F.Cu) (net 5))
 (segment (start 45.085 35.56) (end 46.168 36.643) (width 0.3048) (layer F.Cu) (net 5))
 (segment (start 37.024 38.1) (end 37.024 38.929) (width 0.3048) (layer B.Cu) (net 5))
 (segment (start 37.024 38.929) (end 37.465 39.37) (width 0.3048) (layer B.Cu) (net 5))
 (segment (start 37.465 39.37) (end 39.37 39.37) (width 0.3048) (layer B.Cu) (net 5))
 (segment (start 39.37 39.37) (end 40.64 38.1) (width 0.3048) (layer B.Cu) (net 5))
 (segment (start 40.64 38.1) (end 40.64 36.83) (width 0.3048) (layer B.Cu) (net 5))
 (segment (start 41.91 35.56) (end 43.2212 35.56) (width 0.3048) (layer B.Cu) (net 5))
 (segment (start 40.64 36.83) (end 41.91 35.56) (width 0.3048) (layer B.Cu) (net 5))
 (segment (start 46.168 38.1) (end 46.168 39.183) (width 0.3048) (layer B.Cu) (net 5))
 (segment (start 46.168 39.183) (end 46.99 40.005) (width 0.3048) (layer B.Cu) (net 5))
 (segment (start 46.99 40.005) (end 47.625 40.005) (width 0.3048) (layer B.Cu) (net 5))
 (segment (start 47.625 40.005) (end 50.8 36.83) (width 0.3048) (layer B.Cu) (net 5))
 (segment (start 67.945 28.575) (end 69.85 26.67) (width 0.3048) (layer B.Cu) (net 5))
 (segment (start 66.753908 28.575) (end 67.945 28.575) (width 0.3048) (layer B.Cu) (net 5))
 (segment (start 60.403908 32.385) (end 62.943908 32.385) (width 0.3048) (layer B.Cu) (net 5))
 (segment (start 62.943908 32.385) (end 66.753908 28.575) (width 0.3048) (layer B.Cu) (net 5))
 (segment (start 55.958908 36.83) (end 60.403908 32.385) (width 0.3048) (layer B.Cu) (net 5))
 (segment (start 50.8 36.83) (end 55.958908 36.83) (width 0.3048) (layer B.Cu) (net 5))
 (segment (start 37.024 38.1) (end 37.024 36.001) (width 0.3048) (layer F.Cu) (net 5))
 (segment (start 37.465 35.56) (end 37.465 33.655) (width 0.3048) (layer F.Cu) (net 5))
 (segment (start 37.024 36.001) (end 37.465 35.56) (width 0.3048) (layer F.Cu) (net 5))
 (segment (start 38.274 38.1) (end 38.274 37.291) (width 0.3048) (layer B.Cu) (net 6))
 (segment (start 41.275 34.29) (end 43.2212 34.29) (width 0.3048) (layer B.Cu) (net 6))
 (via (at 43.2212 34.29) (size 0.8) (drill 0.4) (layers F.Cu B.Cu) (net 6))
 (segment (start 38.274 37.291) (end 41.275 34.29) (width 0.3048) (layer B.Cu) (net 6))
 (segment (start 43.2212 34.29) (end 45.006092 34.29) (width 0.3048) (layer F.Cu) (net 6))
 (segment (start 47.418 36.701908) (end 47.418 38.1) (width 0.3048) (layer F.Cu) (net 6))
 (segment (start 45.006092 34.29) (end 47.418 36.701908) (width 0.3048) (layer F.Cu) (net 6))
 (segment (start 67.31 27.305) (end 67.31 26.67) (width 0.3048) (layer B.Cu) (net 6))
 (segment (start 60.325 31.75) (end 62.865 31.75) (width 0.3048) (layer B.Cu) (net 6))
 (segment (start 55.88 36.195) (end 60.325 31.75) (width 0.3048) (layer B.Cu) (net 6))
 (segment (start 62.865 31.75) (end 67.31 27.305) (width 0.3048) (layer B.Cu) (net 6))
 (segment (start 49.323 36.195) (end 55.88 36.195) (width 0.3048) (layer B.Cu) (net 6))
 (segment (start 47.418 38.1) (end 49.323 36.195) (width 0.3048) (layer B.Cu) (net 6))
 (segment (start 38.274 36.021) (end 40.64 33.655) (width 0.3048) (layer F.Cu) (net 6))
 (segment (start 38.274 38.1) (end 38.274 36.021) (width 0.3048) (layer F.Cu) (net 6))
 (segment (start 61.976 38.1) (end 61.976 41.529) (width 0.4064) (layer F.Cu) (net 12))
 (segment (start 61.976 41.529) (end 60.325 43.18) (width 0.4064) (layer F.Cu) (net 12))
 (segment (start 60.325 43.18) (end 52.705 43.18) (width 0.4064) (layer F.Cu) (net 12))
 (segment (start 51.562 42.037) (end 51.562 38.1) (width 0.4064) (layer F.Cu) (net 12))
 (segment (start 52.705 43.18) (end 51.562 42.037) (width 0.4064) (layer F.Cu) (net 12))
 (segment (start 51.562 38.1) (end 51.562 41.783) (width 0.4064) (layer F.Cu) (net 12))
 (segment (start 51.562 41.783) (end 50.165 43.18) (width 0.4064) (layer F.Cu) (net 12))
 (segment (start 50.165 43.18) (end 45.085 43.18) (width 0.4064) (layer F.Cu) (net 12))
 (segment (start 43.668 41.763) (end 43.668 38.1) (width 0.4064) (layer F.Cu) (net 12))
 (segment (start 45.085 43.18) (end 43.668 41.763) (width 0.4064) (layer F.Cu) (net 12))
 (segment (start 43.668 38.1) (end 43.668 38.882) (width 0.4064) (layer B.Cu) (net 12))
 (segment (start 43.668 38.882) (end 42.545 40.005) (width 0.4064) (layer B.Cu) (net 12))
 (segment (start 42.545 40.005) (end 34.925 40.005) (width 0.4064) (layer B.Cu) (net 12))
 (segment (start 34.524 39.604) (end 34.524 38.1) (width 0.4064) (layer B.Cu) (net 12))
 (segment (start 34.925 40.005) (end 34.524 39.604) (width 0.4064) (layer B.Cu) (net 12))
 (segment (start 46.99 26.67) (end 46.99 30.48) (width 0.4064) (layer B.Cu) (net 12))
 (segment (start 46.99 30.48) (end 44.45 33.02) (width 0.4064) (layer B.Cu) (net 12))
 (segment (start 44.45 33.02) (end 44.45 36.195) (width 0.4064) (layer B.Cu) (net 12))
 (segment (start 43.668 36.977) (end 43.668 38.1) (width 0.4064) (layer B.Cu) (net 12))
 (segment (start 44.45 36.195) (end 43.668 36.977) (width 0.4064) (layer B.Cu) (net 12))
 (segment (start 68.476 30.226) (end 66.421 30.226) (width 0.3048) (layer F.Cu) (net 7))
 (segment (start 64.77 28.575) (end 64.77 26.67) (width 0.3048) (layer F.Cu) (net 7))
 (segment (start 66.421 30.226) (end 64.77 28.575) (width 0.3048) (layer F.Cu) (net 7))
 (segment (start 64.77 27.432) (end 64.77 26.67) (width 0.3048) (layer B.Cu) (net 7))
 (segment (start 61.976 30.226) (end 64.77 27.432) (width 0.3048) (layer B.Cu) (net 7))
 (via (at 52.705 34.8076) (size 0.8) (drill 0.4) (layers F.Cu B.Cu) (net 7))
 (segment (start 52.705 33.655) (end 52.705 34.8076) (width 0.3048) (layer F.Cu) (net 7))
 (segment (start 52.705 34.8076) (end 53.574801 35.677401) (width 0.3048) (layer B.Cu) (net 7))
 (segment (start 53.574801 35.677401) (end 55.683691 35.677401) (width 0.3048) (layer B.Cu) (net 7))
 (segment (start 61.135092 30.226) (end 61.976 30.226) (width 0.3048) (layer B.Cu) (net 7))
 (segment (start 55.683691 35.677401) (end 61.135092 30.226) (width 0.3048) (layer B.Cu) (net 7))
 (segment (start 66.976 38.1) (end 66.976 36.94019) (width 0.3048) (layer F.Cu) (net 8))
 (segment (start 66.23081 31.765347) (end 62.405463 27.94) (width 0.3048) (layer F.Cu) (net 8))
 (segment (start 66.23081 36.195) (end 66.23081 31.765347) (width 0.3048) (layer F.Cu) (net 8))
 (segment (start 66.976 36.94019) (end 66.23081 36.195) (width 0.3048) (layer F.Cu) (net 8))
 (segment (start 62.405463 26.845463) (end 62.23 26.67) (width 0.3048) (layer F.Cu) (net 8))
 (segment (start 62.405463 27.94) (end 62.405463 26.845463) (width 0.3048) (layer F.Cu) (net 8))
 (via (at 57.15 30.48) (size 0.8) (drill 0.4) (layers F.Cu B.Cu) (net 3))
 (segment (start 59.69 27.94) (end 57.15 30.48) (width 0.3048) (layer B.Cu) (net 3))
 (segment (start 59.69 26.67) (end 59.69 27.94) (width 0.3048) (layer B.Cu) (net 3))
 (segment (start 57.15 30.48) (end 35.56 30.48) (width 0.3048) (layer F.Cu) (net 3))
 (segment (start 35.56 30.48) (end 31.75 34.29) (width 0.3048) (layer F.Cu) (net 3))
 (segment (start 31.75 34.29) (end 27.94 34.29) (width 0.3048) (layer F.Cu) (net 3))
 (segment (start 65.726 38.1) (end 65.726 35.881) (width 0.3048) (layer F.Cu) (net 9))
 (segment (start 57.15 26.67) (end 57.15 27.94) (width 0.3048) (layer F.Cu) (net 9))
 (segment (start 57.15 27.94) (end 58.083599 28.873599) (width 0.3048) (layer F.Cu) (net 9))
 (segment (start 65.726 31.974446) (end 65.726 35.881) (width 0.3048) (layer F.Cu) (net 9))
 (segment (start 62.625153 28.873599) (end 65.726 31.974446) (width 0.3048) (layer F.Cu) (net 9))
 (segment (start 58.083599 28.873599) (end 62.625153 28.873599) (width 0.3048) (layer F.Cu) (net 9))
 (via (at 54.61 34.925) (size 0.8) (drill 0.4) (layers F.Cu B.Cu) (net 10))
 (segment (start 56.562 36.877) (end 54.61 34.925) (width 0.3048) (layer F.Cu) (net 10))
 (segment (start 56.562 38.1) (end 56.562 36.877) (width 0.3048) (layer F.Cu) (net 10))
 (segment (start 54.61 34.925) (end 54.61 26.67) (width 0.3048) (layer B.Cu) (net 10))
 (segment (start 55.312 37.1452) (end 53.7268 35.56) (width 0.3048) (layer F.Cu) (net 11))
 (segment (start 55.312 38.1) (end 55.312 37.1452) (width 0.3048) (layer F.Cu) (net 11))
 (via (at 50.8 34.925) (size 0.8) (drill 0.4) (layers F.Cu B.Cu) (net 11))
 (segment (start 51.435 35.56) (end 50.8 34.925) (width 0.3048) (layer F.Cu) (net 11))
 (segment (start 53.7268 35.56) (end 51.435 35.56) (width 0.3048) (layer F.Cu) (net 11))
 (segment (start 50.8 34.925) (end 50.8 31.115) (width 0.3048) (layer B.Cu) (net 11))
 (segment (start 52.07 29.845) (end 52.07 26.67) (width 0.3048) (layer B.Cu) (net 11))
 (segment (start 50.8 31.115) (end 52.07 29.845) (width 0.3048) (layer B.Cu) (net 11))
 (segment (start 47.625 33.97) (end 47.625 31.75) (width 0.3048) (layer B.Cu) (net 4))
 (segment (start 49.53 29.845) (end 49.53 26.67) (width 0.3048) (layer B.Cu) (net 4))
 (segment (start 47.625 31.75) (end 49.53 29.845) (width 0.3048) (layer B.Cu) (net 4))
 (segment (start 72.39 36.322) (end 72.39 37.465) (width 0.3048) (layer F.Cu) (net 29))
 (segment (start 74.215 39.29) (end 74.215 40.64) (width 0.3048) (layer F.Cu) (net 29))
 (segment (start 72.39 37.465) (end 74.215 39.29) (width 0.3048) (layer F.Cu) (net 29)))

